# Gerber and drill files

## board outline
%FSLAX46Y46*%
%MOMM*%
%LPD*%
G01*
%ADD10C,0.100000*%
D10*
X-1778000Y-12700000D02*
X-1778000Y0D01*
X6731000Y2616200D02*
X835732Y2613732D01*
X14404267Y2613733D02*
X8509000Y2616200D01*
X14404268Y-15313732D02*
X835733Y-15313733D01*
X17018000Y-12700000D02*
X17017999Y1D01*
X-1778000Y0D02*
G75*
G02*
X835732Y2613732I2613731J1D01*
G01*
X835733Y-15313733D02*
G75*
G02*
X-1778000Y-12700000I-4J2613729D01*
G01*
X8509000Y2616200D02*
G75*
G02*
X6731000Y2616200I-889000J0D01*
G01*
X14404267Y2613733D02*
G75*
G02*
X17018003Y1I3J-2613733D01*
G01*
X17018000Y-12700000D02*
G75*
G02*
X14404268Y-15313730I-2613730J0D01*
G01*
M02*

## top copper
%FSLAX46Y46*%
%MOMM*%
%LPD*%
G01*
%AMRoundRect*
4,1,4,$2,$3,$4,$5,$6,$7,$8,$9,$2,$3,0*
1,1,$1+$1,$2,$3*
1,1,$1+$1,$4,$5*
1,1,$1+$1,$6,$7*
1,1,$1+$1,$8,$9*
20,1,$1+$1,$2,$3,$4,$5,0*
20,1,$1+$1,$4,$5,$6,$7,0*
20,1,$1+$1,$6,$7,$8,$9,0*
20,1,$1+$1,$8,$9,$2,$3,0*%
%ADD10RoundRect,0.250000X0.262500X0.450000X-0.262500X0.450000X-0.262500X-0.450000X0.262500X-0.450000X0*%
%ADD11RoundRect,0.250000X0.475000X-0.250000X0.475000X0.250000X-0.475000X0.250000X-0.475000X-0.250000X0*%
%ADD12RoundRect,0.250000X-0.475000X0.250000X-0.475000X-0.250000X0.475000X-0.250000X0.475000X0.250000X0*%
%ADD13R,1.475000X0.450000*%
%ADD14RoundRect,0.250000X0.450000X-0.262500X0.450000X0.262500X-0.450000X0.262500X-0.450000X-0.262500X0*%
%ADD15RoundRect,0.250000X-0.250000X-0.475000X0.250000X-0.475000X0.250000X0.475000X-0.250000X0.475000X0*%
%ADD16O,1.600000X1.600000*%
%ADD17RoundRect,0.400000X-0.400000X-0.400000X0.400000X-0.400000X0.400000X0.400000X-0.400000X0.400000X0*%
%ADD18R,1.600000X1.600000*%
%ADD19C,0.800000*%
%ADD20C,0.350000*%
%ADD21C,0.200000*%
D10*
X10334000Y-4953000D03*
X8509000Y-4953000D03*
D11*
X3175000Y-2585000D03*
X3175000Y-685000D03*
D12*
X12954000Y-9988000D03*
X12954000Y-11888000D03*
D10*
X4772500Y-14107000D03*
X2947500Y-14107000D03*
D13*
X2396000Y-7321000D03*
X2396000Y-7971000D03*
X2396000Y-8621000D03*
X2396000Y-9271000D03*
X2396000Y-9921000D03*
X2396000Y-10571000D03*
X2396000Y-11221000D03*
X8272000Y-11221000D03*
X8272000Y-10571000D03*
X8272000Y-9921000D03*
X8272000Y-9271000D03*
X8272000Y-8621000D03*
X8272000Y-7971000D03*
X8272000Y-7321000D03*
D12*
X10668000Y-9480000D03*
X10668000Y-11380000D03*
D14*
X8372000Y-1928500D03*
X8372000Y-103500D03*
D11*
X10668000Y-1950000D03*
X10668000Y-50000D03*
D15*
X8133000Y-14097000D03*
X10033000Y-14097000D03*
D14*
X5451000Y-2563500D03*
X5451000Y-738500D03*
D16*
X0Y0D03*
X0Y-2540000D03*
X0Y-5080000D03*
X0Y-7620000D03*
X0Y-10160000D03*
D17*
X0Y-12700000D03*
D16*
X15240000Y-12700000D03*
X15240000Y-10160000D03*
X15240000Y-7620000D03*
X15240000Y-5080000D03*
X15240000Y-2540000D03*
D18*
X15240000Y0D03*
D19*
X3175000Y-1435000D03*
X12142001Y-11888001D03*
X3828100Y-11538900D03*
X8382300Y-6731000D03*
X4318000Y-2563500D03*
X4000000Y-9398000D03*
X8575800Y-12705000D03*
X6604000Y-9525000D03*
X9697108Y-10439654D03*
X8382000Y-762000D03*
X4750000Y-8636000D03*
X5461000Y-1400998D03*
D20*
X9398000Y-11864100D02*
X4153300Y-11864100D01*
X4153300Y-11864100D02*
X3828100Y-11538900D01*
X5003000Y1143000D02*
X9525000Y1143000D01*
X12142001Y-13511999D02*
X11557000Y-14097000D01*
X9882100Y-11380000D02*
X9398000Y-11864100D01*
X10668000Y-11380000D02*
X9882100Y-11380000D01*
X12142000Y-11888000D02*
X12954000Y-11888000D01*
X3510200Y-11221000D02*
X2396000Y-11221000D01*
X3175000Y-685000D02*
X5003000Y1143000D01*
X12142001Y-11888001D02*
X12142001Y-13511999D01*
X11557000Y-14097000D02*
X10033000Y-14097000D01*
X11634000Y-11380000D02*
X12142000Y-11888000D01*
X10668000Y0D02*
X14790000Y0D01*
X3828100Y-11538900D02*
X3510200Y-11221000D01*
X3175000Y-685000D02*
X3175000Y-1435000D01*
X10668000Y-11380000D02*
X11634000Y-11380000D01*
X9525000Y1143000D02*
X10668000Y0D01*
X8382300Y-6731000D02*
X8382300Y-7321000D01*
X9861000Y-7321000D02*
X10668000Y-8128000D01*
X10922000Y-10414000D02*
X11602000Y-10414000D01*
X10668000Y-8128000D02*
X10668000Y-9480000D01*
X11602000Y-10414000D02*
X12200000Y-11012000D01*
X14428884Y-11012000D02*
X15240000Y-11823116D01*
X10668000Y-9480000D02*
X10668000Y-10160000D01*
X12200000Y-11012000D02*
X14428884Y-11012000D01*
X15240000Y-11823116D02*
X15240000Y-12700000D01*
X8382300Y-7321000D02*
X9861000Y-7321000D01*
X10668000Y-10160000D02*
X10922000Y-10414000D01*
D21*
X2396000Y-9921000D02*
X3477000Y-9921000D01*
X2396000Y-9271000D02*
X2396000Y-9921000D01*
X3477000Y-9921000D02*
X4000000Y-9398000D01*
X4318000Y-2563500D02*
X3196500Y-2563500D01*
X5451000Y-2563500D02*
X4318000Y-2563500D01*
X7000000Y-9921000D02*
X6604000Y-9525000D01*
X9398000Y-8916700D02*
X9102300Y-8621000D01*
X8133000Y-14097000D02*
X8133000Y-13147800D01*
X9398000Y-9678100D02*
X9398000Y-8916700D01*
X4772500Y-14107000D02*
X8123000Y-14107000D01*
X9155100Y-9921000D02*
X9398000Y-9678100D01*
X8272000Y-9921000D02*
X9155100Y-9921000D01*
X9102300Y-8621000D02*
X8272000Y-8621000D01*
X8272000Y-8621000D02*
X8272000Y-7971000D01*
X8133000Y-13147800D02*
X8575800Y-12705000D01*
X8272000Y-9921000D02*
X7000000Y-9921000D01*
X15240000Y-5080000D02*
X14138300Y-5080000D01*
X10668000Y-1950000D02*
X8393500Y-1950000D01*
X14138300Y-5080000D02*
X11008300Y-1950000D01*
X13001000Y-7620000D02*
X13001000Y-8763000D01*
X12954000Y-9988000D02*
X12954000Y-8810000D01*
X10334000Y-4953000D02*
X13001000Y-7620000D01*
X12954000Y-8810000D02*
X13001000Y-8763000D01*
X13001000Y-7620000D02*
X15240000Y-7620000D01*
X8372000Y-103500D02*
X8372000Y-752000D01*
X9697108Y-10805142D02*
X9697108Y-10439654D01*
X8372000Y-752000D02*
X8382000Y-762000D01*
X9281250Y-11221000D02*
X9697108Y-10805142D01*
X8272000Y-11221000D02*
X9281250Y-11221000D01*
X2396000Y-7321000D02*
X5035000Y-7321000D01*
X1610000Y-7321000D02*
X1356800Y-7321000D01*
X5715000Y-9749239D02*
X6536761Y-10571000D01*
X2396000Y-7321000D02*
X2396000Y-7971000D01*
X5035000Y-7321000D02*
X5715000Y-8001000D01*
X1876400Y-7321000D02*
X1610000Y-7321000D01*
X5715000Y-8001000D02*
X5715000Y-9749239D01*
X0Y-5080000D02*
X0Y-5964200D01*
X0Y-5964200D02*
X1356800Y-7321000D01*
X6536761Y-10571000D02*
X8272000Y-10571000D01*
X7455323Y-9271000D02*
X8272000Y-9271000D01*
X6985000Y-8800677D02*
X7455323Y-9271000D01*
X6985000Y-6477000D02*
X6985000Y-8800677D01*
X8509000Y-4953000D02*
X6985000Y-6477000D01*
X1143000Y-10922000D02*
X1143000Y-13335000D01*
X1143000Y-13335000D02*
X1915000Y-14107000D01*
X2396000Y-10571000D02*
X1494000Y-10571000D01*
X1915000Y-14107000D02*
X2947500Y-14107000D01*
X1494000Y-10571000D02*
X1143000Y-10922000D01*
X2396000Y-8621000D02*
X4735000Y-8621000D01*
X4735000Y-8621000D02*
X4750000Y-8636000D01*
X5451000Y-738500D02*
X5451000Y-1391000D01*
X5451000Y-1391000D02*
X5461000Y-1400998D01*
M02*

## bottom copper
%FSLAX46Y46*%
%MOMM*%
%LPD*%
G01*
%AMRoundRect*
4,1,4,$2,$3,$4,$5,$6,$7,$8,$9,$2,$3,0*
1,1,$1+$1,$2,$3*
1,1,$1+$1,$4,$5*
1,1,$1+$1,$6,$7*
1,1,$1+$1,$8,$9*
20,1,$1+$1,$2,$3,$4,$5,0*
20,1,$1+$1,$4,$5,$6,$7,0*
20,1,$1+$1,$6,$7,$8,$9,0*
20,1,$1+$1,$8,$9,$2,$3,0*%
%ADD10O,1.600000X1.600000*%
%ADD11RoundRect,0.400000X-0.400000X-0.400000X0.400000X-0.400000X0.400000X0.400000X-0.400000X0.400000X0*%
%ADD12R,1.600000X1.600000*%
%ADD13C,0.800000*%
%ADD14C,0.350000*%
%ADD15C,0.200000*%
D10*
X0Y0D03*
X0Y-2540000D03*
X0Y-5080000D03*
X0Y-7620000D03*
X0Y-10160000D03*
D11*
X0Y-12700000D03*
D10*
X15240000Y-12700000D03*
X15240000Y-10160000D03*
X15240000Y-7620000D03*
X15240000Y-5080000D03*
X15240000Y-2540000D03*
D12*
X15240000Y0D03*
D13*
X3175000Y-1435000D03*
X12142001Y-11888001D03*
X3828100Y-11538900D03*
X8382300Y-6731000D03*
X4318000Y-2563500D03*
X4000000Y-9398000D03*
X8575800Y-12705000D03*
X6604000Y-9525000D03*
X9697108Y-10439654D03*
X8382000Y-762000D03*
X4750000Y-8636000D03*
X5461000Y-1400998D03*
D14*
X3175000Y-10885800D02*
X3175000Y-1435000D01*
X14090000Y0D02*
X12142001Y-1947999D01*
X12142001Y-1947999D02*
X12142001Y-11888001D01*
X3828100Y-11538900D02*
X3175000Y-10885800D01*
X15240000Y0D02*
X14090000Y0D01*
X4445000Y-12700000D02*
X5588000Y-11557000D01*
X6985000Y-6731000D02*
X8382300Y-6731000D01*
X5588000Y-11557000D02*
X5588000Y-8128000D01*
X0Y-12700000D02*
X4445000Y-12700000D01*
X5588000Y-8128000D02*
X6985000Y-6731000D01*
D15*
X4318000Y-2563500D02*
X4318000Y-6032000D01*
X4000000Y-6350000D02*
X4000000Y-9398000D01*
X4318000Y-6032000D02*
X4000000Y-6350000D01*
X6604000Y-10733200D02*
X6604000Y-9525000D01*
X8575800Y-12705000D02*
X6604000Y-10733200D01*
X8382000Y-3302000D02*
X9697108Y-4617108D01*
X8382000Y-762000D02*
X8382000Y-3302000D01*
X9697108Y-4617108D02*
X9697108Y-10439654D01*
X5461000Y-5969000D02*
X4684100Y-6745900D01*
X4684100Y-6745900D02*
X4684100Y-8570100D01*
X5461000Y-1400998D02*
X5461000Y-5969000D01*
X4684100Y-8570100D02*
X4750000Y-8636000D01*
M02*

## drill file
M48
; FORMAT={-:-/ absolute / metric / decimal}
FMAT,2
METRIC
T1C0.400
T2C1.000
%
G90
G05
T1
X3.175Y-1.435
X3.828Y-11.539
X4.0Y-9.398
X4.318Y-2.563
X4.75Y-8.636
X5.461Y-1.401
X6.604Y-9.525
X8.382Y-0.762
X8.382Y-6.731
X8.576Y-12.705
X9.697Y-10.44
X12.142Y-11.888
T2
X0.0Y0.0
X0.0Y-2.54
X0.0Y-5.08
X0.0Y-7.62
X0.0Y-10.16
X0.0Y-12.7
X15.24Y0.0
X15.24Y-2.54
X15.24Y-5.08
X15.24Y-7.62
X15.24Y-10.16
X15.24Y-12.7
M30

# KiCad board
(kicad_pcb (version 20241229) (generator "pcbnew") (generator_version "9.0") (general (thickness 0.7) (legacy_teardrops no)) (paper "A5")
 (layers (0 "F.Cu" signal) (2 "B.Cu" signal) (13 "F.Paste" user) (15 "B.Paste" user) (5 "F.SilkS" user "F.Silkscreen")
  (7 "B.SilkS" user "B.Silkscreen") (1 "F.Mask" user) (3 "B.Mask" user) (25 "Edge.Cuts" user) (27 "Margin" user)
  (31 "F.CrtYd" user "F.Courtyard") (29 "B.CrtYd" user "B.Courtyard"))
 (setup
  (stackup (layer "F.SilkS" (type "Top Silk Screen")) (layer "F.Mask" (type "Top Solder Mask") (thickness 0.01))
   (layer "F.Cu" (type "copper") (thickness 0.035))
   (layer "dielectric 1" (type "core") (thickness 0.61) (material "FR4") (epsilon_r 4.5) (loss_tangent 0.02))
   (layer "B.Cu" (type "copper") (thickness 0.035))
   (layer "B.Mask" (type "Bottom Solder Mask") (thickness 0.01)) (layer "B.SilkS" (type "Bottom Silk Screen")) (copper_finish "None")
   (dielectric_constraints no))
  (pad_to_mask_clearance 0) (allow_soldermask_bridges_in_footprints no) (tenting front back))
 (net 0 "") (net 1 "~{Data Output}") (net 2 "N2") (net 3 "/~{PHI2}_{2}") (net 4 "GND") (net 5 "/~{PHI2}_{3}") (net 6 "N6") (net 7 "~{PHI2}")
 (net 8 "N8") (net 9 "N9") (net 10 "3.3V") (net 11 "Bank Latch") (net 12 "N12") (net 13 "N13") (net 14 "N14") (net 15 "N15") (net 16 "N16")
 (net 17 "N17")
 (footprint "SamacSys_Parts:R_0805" (layer "F.Cu") (at 9.4215 4.943 90)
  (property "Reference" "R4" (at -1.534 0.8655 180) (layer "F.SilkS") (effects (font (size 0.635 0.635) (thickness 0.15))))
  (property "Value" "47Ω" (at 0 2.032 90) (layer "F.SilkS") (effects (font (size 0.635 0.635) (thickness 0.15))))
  (pad "1" smd roundrect (at -0.01 0.9125 180) (size 1.025 1.4) (layers "F.Cu" "F.Mask" "F.Paste") (roundrect_rratio 0.243902)
   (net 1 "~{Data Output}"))
  (pad "2" smd roundrect (at -0.01 -0.9125 180) (size 1.025 1.4) (layers "F.Cu" "F.Mask" "F.Paste") (roundrect_rratio 0.243902) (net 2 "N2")))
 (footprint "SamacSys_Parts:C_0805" (layer "F.Cu") (at 3.175 1.651)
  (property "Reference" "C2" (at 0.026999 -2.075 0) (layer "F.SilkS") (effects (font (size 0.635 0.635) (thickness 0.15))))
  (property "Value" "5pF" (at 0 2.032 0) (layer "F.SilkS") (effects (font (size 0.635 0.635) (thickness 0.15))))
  (pad "1" smd roundrect (at 0 0.934 90) (size 1 1.45) (layers "F.Cu" "F.Mask" "F.Paste") (roundrect_rratio 0.25) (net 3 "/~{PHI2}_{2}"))
  (pad "2" smd roundrect (at 0 -0.966 90) (size 1 1.45) (layers "F.Cu" "F.Mask" "F.Paste") (roundrect_rratio 0.25) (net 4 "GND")))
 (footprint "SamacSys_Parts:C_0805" (layer "F.Cu") (at 12.954 10.922 180)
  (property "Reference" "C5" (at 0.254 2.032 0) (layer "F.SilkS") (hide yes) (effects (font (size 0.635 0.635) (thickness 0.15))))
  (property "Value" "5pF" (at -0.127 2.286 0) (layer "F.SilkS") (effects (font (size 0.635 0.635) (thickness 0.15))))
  (pad "1" smd roundrect (at 0 0.934 270) (size 1 1.45) (layers "F.Cu" "F.Mask" "F.Paste") (roundrect_rratio 0.25) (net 1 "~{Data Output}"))
  (pad "2" smd roundrect (at 0 -0.966 270) (size 1 1.45) (layers "F.Cu" "F.Mask" "F.Paste") (roundrect_rratio 0.25) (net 4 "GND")))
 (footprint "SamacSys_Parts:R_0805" (layer "F.Cu") (at 3.86 14.097 90)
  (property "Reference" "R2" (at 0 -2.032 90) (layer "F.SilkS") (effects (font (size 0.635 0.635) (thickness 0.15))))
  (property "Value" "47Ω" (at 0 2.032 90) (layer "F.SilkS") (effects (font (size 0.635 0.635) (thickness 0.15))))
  (pad "1" smd roundrect (at -0.01 0.9125 180) (size 1.025 1.4) (layers "F.Cu" "F.Mask" "F.Paste") (roundrect_rratio 0.243902)
   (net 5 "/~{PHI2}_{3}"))
  (pad "2" smd roundrect (at -0.01 -0.9125 180) (size 1.025 1.4) (layers "F.Cu" "F.Mask" "F.Paste") (roundrect_rratio 0.243902) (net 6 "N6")))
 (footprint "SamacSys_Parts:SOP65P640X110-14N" (layer "F.Cu") (at 5.334 9.271)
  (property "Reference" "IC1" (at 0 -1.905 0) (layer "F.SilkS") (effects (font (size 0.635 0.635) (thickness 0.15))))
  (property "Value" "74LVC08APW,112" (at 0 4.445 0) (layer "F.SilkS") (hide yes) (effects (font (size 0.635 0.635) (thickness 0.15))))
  (pad "1" smd rect (at -2.938 -1.95 90) (size 0.45 1.475) (layers "F.Cu" "F.Mask" "F.Paste") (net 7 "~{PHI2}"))
  (pad "2" smd rect (at -2.938 -1.3 90) (size 0.45 1.475) (layers "F.Cu" "F.Mask" "F.Paste") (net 7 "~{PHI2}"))
  (pad "3" smd rect (at -2.938 -0.65 90) (size 0.45 1.475) (layers "F.Cu" "F.Mask" "F.Paste") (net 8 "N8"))
  (pad "4" smd rect (at -2.938 0 90) (size 0.45 1.475) (layers "F.Cu" "F.Mask" "F.Paste") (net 3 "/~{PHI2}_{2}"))
  (pad "5" smd rect (at -2.938 0.65 90) (size 0.45 1.475) (layers "F.Cu" "F.Mask" "F.Paste") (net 3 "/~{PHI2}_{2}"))
  (pad "6" smd rect (at -2.938 1.3 90) (size 0.45 1.475) (layers "F.Cu" "F.Mask" "F.Paste") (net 6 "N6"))
  (pad "7" smd rect (at -2.938 1.95 90) (size 0.45 1.475) (layers "F.Cu" "F.Mask" "F.Paste") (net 4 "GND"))
  (pad "8" smd rect (at 2.938 1.95 90) (size 0.45 1.475) (layers "F.Cu" "F.Mask" "F.Paste") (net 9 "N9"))
  (pad "9" smd rect (at 2.938 1.3 90) (size 0.45 1.475) (layers "F.Cu" "F.Mask" "F.Paste") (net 7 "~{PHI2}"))
  (pad "10" smd rect (at 2.938 0.65 90) (size 0.45 1.475) (layers "F.Cu" "F.Mask" "F.Paste") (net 5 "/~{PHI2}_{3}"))
  (pad "11" smd rect (at 2.938 0 90) (size 0.45 1.475) (layers "F.Cu" "F.Mask" "F.Paste") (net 2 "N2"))
  (pad "12" smd rect (at 2.938 -0.65 90) (size 0.45 1.475) (layers "F.Cu" "F.Mask" "F.Paste") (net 5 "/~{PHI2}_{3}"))
  (pad "13" smd rect (at 2.938 -1.3 90) (size 0.45 1.475) (layers "F.Cu" "F.Mask" "F.Paste") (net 5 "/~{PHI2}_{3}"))
  (pad "14" smd rect (at 2.938 -1.95 90) (size 0.45 1.475) (layers "F.Cu" "F.Mask" "F.Paste") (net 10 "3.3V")))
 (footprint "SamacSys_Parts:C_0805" (layer "F.Cu") (at 10.668 10.414 180)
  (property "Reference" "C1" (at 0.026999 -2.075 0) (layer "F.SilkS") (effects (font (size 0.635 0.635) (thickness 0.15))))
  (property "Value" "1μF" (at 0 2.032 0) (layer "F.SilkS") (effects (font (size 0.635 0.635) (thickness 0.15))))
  (pad "1" smd roundrect (at 0 0.934 270) (size 1 1.45) (layers "F.Cu" "F.Mask" "F.Paste") (roundrect_rratio 0.25) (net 10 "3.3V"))
  (pad "2" smd roundrect (at 0 -0.966 270) (size 1 1.45) (layers "F.Cu" "F.Mask" "F.Paste") (roundrect_rratio 0.25) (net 4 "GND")))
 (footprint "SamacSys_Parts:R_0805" (layer "F.Cu") (at 8.382 1.016)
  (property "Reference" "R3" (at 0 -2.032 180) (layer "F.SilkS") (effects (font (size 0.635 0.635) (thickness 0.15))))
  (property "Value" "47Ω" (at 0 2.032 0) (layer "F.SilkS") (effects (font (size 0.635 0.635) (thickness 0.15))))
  (pad "1" smd roundrect (at -0.01 0.9125 90) (size 1.025 1.4) (layers "F.Cu" "F.Mask" "F.Paste") (roundrect_rratio 0.243902)
   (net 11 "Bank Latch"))
  (pad "2" smd roundrect (at -0.01 -0.9125 90) (size 1.025 1.4) (layers "F.Cu" "F.Mask" "F.Paste") (roundrect_rratio 0.243902) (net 9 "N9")))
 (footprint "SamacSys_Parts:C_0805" (layer "F.Cu") (at 10.668 1.016)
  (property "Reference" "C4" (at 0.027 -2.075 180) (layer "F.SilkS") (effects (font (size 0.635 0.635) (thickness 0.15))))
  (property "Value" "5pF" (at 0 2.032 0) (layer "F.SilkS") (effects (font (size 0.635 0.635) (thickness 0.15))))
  (pad "1" smd roundrect (at 0 0.934 90) (size 1 1.45) (layers "F.Cu" "F.Mask" "F.Paste") (roundrect_rratio 0.25) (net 11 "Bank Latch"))
  (pad "2" smd roundrect (at 0 -0.966 90) (size 1 1.45) (layers "F.Cu" "F.Mask" "F.Paste") (roundrect_rratio 0.25) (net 4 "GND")))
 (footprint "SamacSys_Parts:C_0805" (layer "F.Cu") (at 9.067 14.097 -90)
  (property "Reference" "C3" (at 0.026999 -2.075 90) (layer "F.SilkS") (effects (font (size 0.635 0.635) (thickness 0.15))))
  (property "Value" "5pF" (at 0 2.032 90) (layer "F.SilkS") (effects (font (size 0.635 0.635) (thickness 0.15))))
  (pad "1" smd roundrect (at 0 0.934) (size 1 1.45) (layers "F.Cu" "F.Mask" "F.Paste") (roundrect_rratio 0.25) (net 5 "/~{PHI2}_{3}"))
  (pad "2" smd roundrect (at 0 -0.966) (size 1 1.45) (layers "F.Cu" "F.Mask" "F.Paste") (roundrect_rratio 0.25) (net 4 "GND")))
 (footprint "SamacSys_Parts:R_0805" (layer "F.Cu") (at 5.461 1.651)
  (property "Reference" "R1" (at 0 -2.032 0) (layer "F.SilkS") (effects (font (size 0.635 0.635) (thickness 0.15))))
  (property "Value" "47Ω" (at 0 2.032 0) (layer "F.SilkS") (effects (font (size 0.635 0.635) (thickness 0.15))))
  (pad "1" smd roundrect (at -0.01 0.9125 90) (size 1.025 1.4) (layers "F.Cu" "F.Mask" "F.Paste") (roundrect_rratio 0.243902)
   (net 3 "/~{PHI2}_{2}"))
  (pad "2" smd roundrect (at -0.01 -0.9125 90) (size 1.025 1.4) (layers "F.Cu" "F.Mask" "F.Paste") (roundrect_rratio 0.243902) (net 8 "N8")))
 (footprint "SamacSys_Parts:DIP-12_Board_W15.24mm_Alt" (layer "F.Cu") (at 0 0)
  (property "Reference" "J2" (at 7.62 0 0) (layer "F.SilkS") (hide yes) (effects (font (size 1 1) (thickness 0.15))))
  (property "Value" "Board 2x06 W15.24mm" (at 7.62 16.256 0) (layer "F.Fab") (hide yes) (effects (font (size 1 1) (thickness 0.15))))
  (fp_line (start -1.778 12.7) (end -1.778 0) (stroke (width 0.1) (type solid)) (layer "Edge.Cuts"))
  (fp_line (start 6.731 -2.6162) (end 0.835732 -2.613732) (stroke (width 0.1) (type solid)) (layer "Edge.Cuts"))
  (fp_line (start 14.404267 -2.613733) (end 8.509 -2.6162) (stroke (width 0.1) (type solid)) (layer "Edge.Cuts"))
  (fp_line (start 14.404268 15.313732) (end 0.835733 15.313733) (stroke (width 0.1) (type solid)) (layer "Edge.Cuts"))
  (fp_line (start 17.018 12.7) (end 17.017999 -0.000001) (stroke (width 0.1) (type solid)) (layer "Edge.Cuts"))
  (fp_arc (start -1.778 0) (mid -1.012456 -1.848188) (end 0.835732 -2.613732) (stroke (width 0.1) (type solid)) (layer "Edge.Cuts"))
  (fp_arc (start 0.835733 15.313733) (mid -1.012457 14.548189) (end -1.778 12.7) (stroke (width 0.1) (type solid)) (layer "Edge.Cuts"))
  (fp_arc (start 8.509 -2.6162) (mid 7.62 -1.7272) (end 6.731 -2.6162) (stroke (width 0.1) (type default)) (layer "Edge.Cuts"))
  (fp_arc (start 14.404267 -2.613733) (mid 16.252455 -1.848189) (end 17.017999 -0.000001) (stroke (width 0.1) (type solid))
   (layer "Edge.Cuts"))
  (fp_arc (start 17.018 12.7) (mid 16.252456 14.548187) (end 14.404268 15.313732) (stroke (width 0.1) (type solid)) (layer "Edge.Cuts"))
  (pad "1" thru_hole oval (at 0 0 180) (size 1.6 1.6) (drill 1) (layers "*.Cu" "*.Mask") (remove_unused_layers no) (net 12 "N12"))
  (pad "2" thru_hole oval (at 0 2.54) (size 1.6 1.6) (drill 1) (layers "*.Cu" "*.Mask") (remove_unused_layers no) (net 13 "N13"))
  (pad "3" thru_hole oval (at 0 5.08) (size 1.6 1.6) (drill 1) (layers "*.Cu" "*.Mask") (remove_unused_layers no) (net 7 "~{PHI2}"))
  (pad "4" thru_hole oval (at 0 7.62 180) (size 1.6 1.6) (drill 1) (layers "*.Cu" "*.Mask") (remove_unused_layers no) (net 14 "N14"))
  (pad "5" thru_hole oval (at 0 10.16) (size 1.6 1.6) (drill 1) (layers "*.Cu" "*.Mask") (remove_unused_layers no) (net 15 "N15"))
  (pad "6" thru_hole roundrect (at 0 12.7) (size 1.6 1.6) (drill 1) (layers "*.Cu" "*.Mask") (remove_unused_layers no)
   (roundrect_rratio 0.25) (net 10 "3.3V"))
  (pad "7" thru_hole oval (at 15.24 12.7 180) (size 1.6 1.6) (drill 1) (layers "*.Cu" "*.Mask") (remove_unused_layers no) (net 10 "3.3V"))
  (pad "8" thru_hole oval (at 15.24 10.16 180) (size 1.6 1.6) (drill 1) (layers "*.Cu" "*.Mask") (remove_unused_layers no) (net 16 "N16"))
  (pad "9" thru_hole oval (at 15.24 7.62 180) (size 1.6 1.6) (drill 1) (layers "*.Cu" "*.Mask") (remove_unused_layers no)
   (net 1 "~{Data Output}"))
  (pad "10" thru_hole oval (at 15.24 5.08) (size 1.6 1.6) (drill 1) (layers "*.Cu" "*.Mask") (remove_unused_layers no) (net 11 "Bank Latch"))
  (pad "11" thru_hole oval (at 15.24 2.54) (size 1.6 1.6) (drill 1) (layers "*.Cu" "*.Mask") (remove_unused_layers no) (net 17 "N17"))
  (pad "12" thru_hole rect (at 15.24 0) (size 1.6 1.6) (drill 1) (layers "*.Cu" "*.Mask") (remove_unused_layers no) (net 4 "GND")))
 (segment (start 9.398 11.8641) (end 4.1533 11.8641) (width 0.35) (layer "F.Cu") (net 4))
 (segment (start 4.1533 11.8641) (end 3.8281 11.5389) (width 0.35) (layer "F.Cu") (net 4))
 (segment (start 5.003 -1.143) (end 9.525 -1.143) (width 0.35) (layer "F.Cu") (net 4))
 (segment (start 12.142001 13.511999) (end 11.557 14.097) (width 0.35) (layer "F.Cu") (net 4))
 (segment (start 9.8821 11.38) (end 9.398 11.8641) (width 0.35) (layer "F.Cu") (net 4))
 (segment (start 10.668 11.38) (end 9.8821 11.38) (width 0.35) (layer "F.Cu") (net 4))
 (segment (start 12.142 11.888) (end 12.954 11.888) (width 0.35) (layer "F.Cu") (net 4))
 (segment (start 3.5102 11.221) (end 2.396 11.221) (width 0.35) (layer "F.Cu") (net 4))
 (segment (start 3.175 0.685) (end 5.003 -1.143) (width 0.35) (layer "F.Cu") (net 4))
 (segment (start 12.142001 11.888001) (end 12.142001 13.511999) (width 0.35) (layer "F.Cu") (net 4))
 (segment (start 11.557 14.097) (end 10.033 14.097) (width 0.35) (layer "F.Cu") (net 4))
 (segment (start 11.634 11.38) (end 12.142 11.888) (width 0.35) (layer "F.Cu") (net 4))
 (segment (start 10.668 0) (end 14.79 0) (width 0.35) (layer "F.Cu") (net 4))
 (segment (start 3.8281 11.5389) (end 3.5102 11.221) (width 0.35) (layer "F.Cu") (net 4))
 (segment (start 3.175 0.685) (end 3.175 1.435) (width 0.35) (layer "F.Cu") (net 4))
 (segment (start 10.668 11.38) (end 11.634 11.38) (width 0.35) (layer "F.Cu") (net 4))
 (segment (start 9.525 -1.143) (end 10.668 0) (width 0.35) (layer "F.Cu") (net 4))
 (via (at 3.175 1.435) (size 0.8) (drill 0.4) (layers "F.Cu" "B.Cu") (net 4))
 (via (at 12.142001 11.888001) (size 0.8) (drill 0.4) (layers "F.Cu" "B.Cu") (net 4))
 (via (at 3.8281 11.5389) (size 0.8) (drill 0.4) (layers "F.Cu" "B.Cu") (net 4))
 (segment (start 3.175 10.8858) (end 3.175 1.435) (width 0.35) (layer "B.Cu") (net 4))
 (segment (start 14.09 0) (end 12.142001 1.947999) (width 0.35) (layer "B.Cu") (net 4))
 (segment (start 12.142001 1.947999) (end 12.142001 11.888001) (width 0.35) (layer "B.Cu") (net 4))
 (segment (start 3.8281 11.5389) (end 3.175 10.8858) (width 0.35) (layer "B.Cu") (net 4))
 (segment (start 15.24 0) (end 14.09 0) (width 0.35) (layer "B.Cu") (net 4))
 (segment (start 8.3823 6.731) (end 8.3823 7.321) (width 0.35) (layer "F.Cu") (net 10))
 (segment (start 9.861 7.321) (end 10.668 8.128) (width 0.35) (layer "F.Cu") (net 10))
 (segment (start 10.922 10.414) (end 11.602 10.414) (width 0.35) (layer "F.Cu") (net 10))
 (segment (start 10.668 8.128) (end 10.668 9.48) (width 0.35) (layer "F.Cu") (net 10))
 (segment (start 11.602 10.414) (end 12.2 11.012) (width 0.35) (layer "F.Cu") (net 10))
 (segment (start 14.428884 11.012) (end 15.24 11.823116) (width 0.35) (layer "F.Cu") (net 10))
 (segment (start 10.668 9.48) (end 10.668 10.16) (width 0.35) (layer "F.Cu") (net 10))
 (segment (start 12.2 11.012) (end 14.428884 11.012) (width 0.35) (layer "F.Cu") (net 10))
 (segment (start 15.24 11.823116) (end 15.24 12.7) (width 0.35) (layer "F.Cu") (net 10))
 (segment (start 8.3823 7.321) (end 9.861 7.321) (width 0.35) (layer "F.Cu") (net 10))
 (segment (start 10.668 10.16) (end 10.922 10.414) (width 0.35) (layer "F.Cu") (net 10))
 (via (at 8.3823 6.731) (size 0.8) (drill 0.4) (layers "F.Cu" "B.Cu") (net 10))
 (segment (start 4.445 12.7) (end 5.588 11.557) (width 0.35) (layer "B.Cu") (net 10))
 (segment (start 6.985 6.731) (end 8.3823 6.731) (width 0.35) (layer "B.Cu") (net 10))
 (segment (start 5.588 11.557) (end 5.588 8.128) (width 0.35) (layer "B.Cu") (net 10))
 (segment (start 0 12.7) (end 4.445 12.7) (width 0.35) (layer "B.Cu") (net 10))
 (segment (start 5.588 8.128) (end 6.985 6.731) (width 0.35) (layer "B.Cu") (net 10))
 (segment (start 2.396 9.921) (end 3.477 9.921) (width 0.2) (layer "F.Cu") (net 3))
 (segment (start 2.396 9.271) (end 2.396 9.921) (width 0.2) (layer "F.Cu") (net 3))
 (segment (start 3.477 9.921) (end 4 9.398) (width 0.2) (layer "F.Cu") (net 3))
 (segment (start 4.318 2.5635) (end 3.1965 2.5635) (width 0.2) (layer "F.Cu") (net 3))
 (segment (start 5.451 2.5635) (end 4.318 2.5635) (width 0.2) (layer "F.Cu") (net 3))
 (via (at 4.318 2.5635) (size 0.8) (drill 0.4) (layers "F.Cu" "B.Cu") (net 3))
 (via (at 4 9.398) (size 0.8) (drill 0.4) (layers "F.Cu" "B.Cu") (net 3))
 (segment (start 4.318 2.5635) (end 4.318 6.032) (width 0.2) (layer "B.Cu") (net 3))
 (segment (start 4 6.35) (end 4 9.398) (width 0.2) (layer "B.Cu") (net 3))
 (segment (start 4.318 6.032) (end 4 6.35) (width 0.2) (layer "B.Cu") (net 3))
 (segment (start 7 9.921) (end 6.604 9.525) (width 0.2) (layer "F.Cu") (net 5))
 (segment (start 9.398 8.9167) (end 9.1023 8.621) (width 0.2) (layer "F.Cu") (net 5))
 (segment (start 8.133 14.097) (end 8.133 13.1478) (width 0.2) (layer "F.Cu") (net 5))
 (segment (start 9.398 9.6781) (end 9.398 8.9167) (width 0.2) (layer "F.Cu") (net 5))
 (segment (start 4.7725 14.107) (end 8.123 14.107) (width 0.2) (layer "F.Cu") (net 5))
 (segment (start 9.1551 9.921) (end 9.398 9.6781) (width 0.2) (layer "F.Cu") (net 5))
 (segment (start 8.272 9.921) (end 9.1551 9.921) (width 0.2) (layer "F.Cu") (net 5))
 (segment (start 9.1023 8.621) (end 8.272 8.621) (width 0.2) (layer "F.Cu") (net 5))
 (segment (start 8.272 8.621) (end 8.272 7.971) (width 0.2) (layer "F.Cu") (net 5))
 (segment (start 8.133 13.1478) (end 8.5758 12.705) (width 0.2) (layer "F.Cu") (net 5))
 (segment (start 8.272 9.921) (end 7 9.921) (width 0.2) (layer "F.Cu") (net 5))
 (via (at 8.5758 12.705) (size 0.8) (drill 0.4) (layers "F.Cu" "B.Cu") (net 5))
 (via (at 6.604 9.525) (size 0.8) (drill 0.4) (layers "F.Cu" "B.Cu") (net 5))
 (segment (start 6.604 10.7332) (end 6.604 9.525) (width 0.2) (layer "B.Cu") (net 5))
 (segment (start 8.5758 12.705) (end 6.604 10.7332) (width 0.2) (layer "B.Cu") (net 5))
 (segment (start 15.24 5.08) (end 14.1383 5.08) (width 0.2) (layer "F.Cu") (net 11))
 (segment (start 10.668 1.95) (end 8.3935 1.95) (width 0.2) (layer "F.Cu") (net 11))
 (segment (start 14.1383 5.08) (end 11.0083 1.95) (width 0.2) (layer "F.Cu") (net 11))
 (segment (start 13.001 7.62) (end 13.001 8.763) (width 0.2) (layer "F.Cu") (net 1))
 (segment (start 12.954 9.988) (end 12.954 8.81) (width 0.2) (layer "F.Cu") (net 1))
 (segment (start 10.334 4.953) (end 13.001 7.62) (width 0.2) (layer "F.Cu") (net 1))
 (segment (start 12.954 8.81) (end 13.001 8.763) (width 0.2) (layer "F.Cu") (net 1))
 (segment (start 13.001 7.62) (end 15.24 7.62) (width 0.2) (layer "F.Cu") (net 1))
 (segment (start 8.372 0.1035) (end 8.372 0.752) (width 0.2) (layer "F.Cu") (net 9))
 (segment (start 9.697108 10.805142) (end 9.697108 10.439654) (width 0.2) (layer "F.Cu") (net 9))
 (segment (start 8.372 0.752) (end 8.382 0.762) (width 0.2) (layer "F.Cu") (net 9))
 (segment (start 9.28125 11.221) (end 9.697108 10.805142) (width 0.2) (layer "F.Cu") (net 9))
 (segment (start 8.272 11.221) (end 9.28125 11.221) (width 0.2) (layer "F.Cu") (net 9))
 (via (at 9.697108 10.439654) (size 0.8) (drill 0.4) (layers "F.Cu" "B.Cu") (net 9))
 (via (at 8.382 0.762) (size 0.8) (drill 0.4) (layers "F.Cu" "B.Cu") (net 9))
 (segment (start 8.382 3.302) (end 9.697108 4.617108) (width 0.2) (layer "B.Cu") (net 9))
 (segment (start 8.382 0.762) (end 8.382 3.302) (width 0.2) (layer "B.Cu") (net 9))
 (segment (start 9.697108 4.617108) (end 9.697108 10.439654) (width 0.2) (layer "B.Cu") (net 9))
 (segment (start 2.396 7.321) (end 5.035 7.321) (width 0.2) (layer "F.Cu") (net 7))
 (segment (start 1.61 7.321) (end 1.3568 7.321) (width 0.2) (layer "F.Cu") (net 7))
 (segment (start 5.715 9.749239) (end 6.536761 10.571) (width 0.2) (layer "F.Cu") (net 7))
 (segment (start 2.396 7.321) (end 2.396 7.971) (width 0.2) (layer "F.Cu") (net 7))
 (segment (start 5.035 7.321) (end 5.715 8.001) (width 0.2) (layer "F.Cu") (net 7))
 (segment (start 1.8764 7.321) (end 1.61 7.321) (width 0.2) (layer "F.Cu") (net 7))
 (segment (start 5.715 8.001) (end 5.715 9.749239) (width 0.2) (layer "F.Cu") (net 7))
 (segment (start 0 5.08) (end 0 5.9642) (width 0.2) (layer "F.Cu") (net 7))
 (segment (start 0 5.9642) (end 1.3568 7.321) (width 0.2) (layer "F.Cu") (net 7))
 (segment (start 6.536761 10.571) (end 8.272 10.571) (width 0.2) (layer "F.Cu") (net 7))
 (segment (start 7.455323 9.271) (end 8.272 9.271) (width 0.2) (layer "F.Cu") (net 2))
 (segment (start 6.985 8.800677) (end 7.455323 9.271) (width 0.2) (layer "F.Cu") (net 2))
 (segment (start 6.985 6.477) (end 6.985 8.800677) (width 0.2) (layer "F.Cu") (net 2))
 (segment (start 8.509 4.953) (end 6.985 6.477) (width 0.2) (layer "F.Cu") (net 2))
 (segment (start 1.143 10.922) (end 1.143 13.335) (width 0.2) (layer "F.Cu") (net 6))
 (segment (start 1.143 13.335) (end 1.915 14.107) (width 0.2) (layer "F.Cu") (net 6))
 (segment (start 2.396 10.571) (end 1.494 10.571) (width 0.2) (layer "F.Cu") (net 6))
 (segment (start 1.915 14.107) (end 2.9475 14.107) (width 0.2) (layer "F.Cu") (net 6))
 (segment (start 1.494 10.571) (end 1.143 10.922) (width 0.2) (layer "F.Cu") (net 6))
 (segment (start 2.396 8.621) (end 4.735 8.621) (width 0.2) (layer "F.Cu") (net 8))
 (segment (start 4.735 8.621) (end 4.75 8.636) (width 0.2) (layer "F.Cu") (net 8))
 (segment (start 5.451 0.7385) (end 5.451 1.391) (width 0.2) (layer "F.Cu") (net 8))
 (segment (start 5.451 1.391) (end 5.461 1.400998) (width 0.2) (layer "F.Cu") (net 8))
 (via (at 4.75 8.636) (size 0.8) (drill 0.4) (layers "F.Cu" "B.Cu") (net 8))
 (via (at 5.461 1.400998) (size 0.8) (drill 0.4) (layers "F.Cu" "B.Cu") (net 8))
 (segment (start 5.461 5.969) (end 4.6841 6.7459) (width 0.2) (layer "B.Cu") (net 8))
 (segment (start 4.6841 6.7459) (end 4.6841 8.5701) (width 0.2) (layer "B.Cu") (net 8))
 (segment (start 5.461 1.400998) (end 5.461 5.969) (width 0.2) (layer "B.Cu") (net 8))
 (segment (start 4.6841 8.5701) (end 4.75 8.636) (width 0.2) (layer "B.Cu") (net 8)))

